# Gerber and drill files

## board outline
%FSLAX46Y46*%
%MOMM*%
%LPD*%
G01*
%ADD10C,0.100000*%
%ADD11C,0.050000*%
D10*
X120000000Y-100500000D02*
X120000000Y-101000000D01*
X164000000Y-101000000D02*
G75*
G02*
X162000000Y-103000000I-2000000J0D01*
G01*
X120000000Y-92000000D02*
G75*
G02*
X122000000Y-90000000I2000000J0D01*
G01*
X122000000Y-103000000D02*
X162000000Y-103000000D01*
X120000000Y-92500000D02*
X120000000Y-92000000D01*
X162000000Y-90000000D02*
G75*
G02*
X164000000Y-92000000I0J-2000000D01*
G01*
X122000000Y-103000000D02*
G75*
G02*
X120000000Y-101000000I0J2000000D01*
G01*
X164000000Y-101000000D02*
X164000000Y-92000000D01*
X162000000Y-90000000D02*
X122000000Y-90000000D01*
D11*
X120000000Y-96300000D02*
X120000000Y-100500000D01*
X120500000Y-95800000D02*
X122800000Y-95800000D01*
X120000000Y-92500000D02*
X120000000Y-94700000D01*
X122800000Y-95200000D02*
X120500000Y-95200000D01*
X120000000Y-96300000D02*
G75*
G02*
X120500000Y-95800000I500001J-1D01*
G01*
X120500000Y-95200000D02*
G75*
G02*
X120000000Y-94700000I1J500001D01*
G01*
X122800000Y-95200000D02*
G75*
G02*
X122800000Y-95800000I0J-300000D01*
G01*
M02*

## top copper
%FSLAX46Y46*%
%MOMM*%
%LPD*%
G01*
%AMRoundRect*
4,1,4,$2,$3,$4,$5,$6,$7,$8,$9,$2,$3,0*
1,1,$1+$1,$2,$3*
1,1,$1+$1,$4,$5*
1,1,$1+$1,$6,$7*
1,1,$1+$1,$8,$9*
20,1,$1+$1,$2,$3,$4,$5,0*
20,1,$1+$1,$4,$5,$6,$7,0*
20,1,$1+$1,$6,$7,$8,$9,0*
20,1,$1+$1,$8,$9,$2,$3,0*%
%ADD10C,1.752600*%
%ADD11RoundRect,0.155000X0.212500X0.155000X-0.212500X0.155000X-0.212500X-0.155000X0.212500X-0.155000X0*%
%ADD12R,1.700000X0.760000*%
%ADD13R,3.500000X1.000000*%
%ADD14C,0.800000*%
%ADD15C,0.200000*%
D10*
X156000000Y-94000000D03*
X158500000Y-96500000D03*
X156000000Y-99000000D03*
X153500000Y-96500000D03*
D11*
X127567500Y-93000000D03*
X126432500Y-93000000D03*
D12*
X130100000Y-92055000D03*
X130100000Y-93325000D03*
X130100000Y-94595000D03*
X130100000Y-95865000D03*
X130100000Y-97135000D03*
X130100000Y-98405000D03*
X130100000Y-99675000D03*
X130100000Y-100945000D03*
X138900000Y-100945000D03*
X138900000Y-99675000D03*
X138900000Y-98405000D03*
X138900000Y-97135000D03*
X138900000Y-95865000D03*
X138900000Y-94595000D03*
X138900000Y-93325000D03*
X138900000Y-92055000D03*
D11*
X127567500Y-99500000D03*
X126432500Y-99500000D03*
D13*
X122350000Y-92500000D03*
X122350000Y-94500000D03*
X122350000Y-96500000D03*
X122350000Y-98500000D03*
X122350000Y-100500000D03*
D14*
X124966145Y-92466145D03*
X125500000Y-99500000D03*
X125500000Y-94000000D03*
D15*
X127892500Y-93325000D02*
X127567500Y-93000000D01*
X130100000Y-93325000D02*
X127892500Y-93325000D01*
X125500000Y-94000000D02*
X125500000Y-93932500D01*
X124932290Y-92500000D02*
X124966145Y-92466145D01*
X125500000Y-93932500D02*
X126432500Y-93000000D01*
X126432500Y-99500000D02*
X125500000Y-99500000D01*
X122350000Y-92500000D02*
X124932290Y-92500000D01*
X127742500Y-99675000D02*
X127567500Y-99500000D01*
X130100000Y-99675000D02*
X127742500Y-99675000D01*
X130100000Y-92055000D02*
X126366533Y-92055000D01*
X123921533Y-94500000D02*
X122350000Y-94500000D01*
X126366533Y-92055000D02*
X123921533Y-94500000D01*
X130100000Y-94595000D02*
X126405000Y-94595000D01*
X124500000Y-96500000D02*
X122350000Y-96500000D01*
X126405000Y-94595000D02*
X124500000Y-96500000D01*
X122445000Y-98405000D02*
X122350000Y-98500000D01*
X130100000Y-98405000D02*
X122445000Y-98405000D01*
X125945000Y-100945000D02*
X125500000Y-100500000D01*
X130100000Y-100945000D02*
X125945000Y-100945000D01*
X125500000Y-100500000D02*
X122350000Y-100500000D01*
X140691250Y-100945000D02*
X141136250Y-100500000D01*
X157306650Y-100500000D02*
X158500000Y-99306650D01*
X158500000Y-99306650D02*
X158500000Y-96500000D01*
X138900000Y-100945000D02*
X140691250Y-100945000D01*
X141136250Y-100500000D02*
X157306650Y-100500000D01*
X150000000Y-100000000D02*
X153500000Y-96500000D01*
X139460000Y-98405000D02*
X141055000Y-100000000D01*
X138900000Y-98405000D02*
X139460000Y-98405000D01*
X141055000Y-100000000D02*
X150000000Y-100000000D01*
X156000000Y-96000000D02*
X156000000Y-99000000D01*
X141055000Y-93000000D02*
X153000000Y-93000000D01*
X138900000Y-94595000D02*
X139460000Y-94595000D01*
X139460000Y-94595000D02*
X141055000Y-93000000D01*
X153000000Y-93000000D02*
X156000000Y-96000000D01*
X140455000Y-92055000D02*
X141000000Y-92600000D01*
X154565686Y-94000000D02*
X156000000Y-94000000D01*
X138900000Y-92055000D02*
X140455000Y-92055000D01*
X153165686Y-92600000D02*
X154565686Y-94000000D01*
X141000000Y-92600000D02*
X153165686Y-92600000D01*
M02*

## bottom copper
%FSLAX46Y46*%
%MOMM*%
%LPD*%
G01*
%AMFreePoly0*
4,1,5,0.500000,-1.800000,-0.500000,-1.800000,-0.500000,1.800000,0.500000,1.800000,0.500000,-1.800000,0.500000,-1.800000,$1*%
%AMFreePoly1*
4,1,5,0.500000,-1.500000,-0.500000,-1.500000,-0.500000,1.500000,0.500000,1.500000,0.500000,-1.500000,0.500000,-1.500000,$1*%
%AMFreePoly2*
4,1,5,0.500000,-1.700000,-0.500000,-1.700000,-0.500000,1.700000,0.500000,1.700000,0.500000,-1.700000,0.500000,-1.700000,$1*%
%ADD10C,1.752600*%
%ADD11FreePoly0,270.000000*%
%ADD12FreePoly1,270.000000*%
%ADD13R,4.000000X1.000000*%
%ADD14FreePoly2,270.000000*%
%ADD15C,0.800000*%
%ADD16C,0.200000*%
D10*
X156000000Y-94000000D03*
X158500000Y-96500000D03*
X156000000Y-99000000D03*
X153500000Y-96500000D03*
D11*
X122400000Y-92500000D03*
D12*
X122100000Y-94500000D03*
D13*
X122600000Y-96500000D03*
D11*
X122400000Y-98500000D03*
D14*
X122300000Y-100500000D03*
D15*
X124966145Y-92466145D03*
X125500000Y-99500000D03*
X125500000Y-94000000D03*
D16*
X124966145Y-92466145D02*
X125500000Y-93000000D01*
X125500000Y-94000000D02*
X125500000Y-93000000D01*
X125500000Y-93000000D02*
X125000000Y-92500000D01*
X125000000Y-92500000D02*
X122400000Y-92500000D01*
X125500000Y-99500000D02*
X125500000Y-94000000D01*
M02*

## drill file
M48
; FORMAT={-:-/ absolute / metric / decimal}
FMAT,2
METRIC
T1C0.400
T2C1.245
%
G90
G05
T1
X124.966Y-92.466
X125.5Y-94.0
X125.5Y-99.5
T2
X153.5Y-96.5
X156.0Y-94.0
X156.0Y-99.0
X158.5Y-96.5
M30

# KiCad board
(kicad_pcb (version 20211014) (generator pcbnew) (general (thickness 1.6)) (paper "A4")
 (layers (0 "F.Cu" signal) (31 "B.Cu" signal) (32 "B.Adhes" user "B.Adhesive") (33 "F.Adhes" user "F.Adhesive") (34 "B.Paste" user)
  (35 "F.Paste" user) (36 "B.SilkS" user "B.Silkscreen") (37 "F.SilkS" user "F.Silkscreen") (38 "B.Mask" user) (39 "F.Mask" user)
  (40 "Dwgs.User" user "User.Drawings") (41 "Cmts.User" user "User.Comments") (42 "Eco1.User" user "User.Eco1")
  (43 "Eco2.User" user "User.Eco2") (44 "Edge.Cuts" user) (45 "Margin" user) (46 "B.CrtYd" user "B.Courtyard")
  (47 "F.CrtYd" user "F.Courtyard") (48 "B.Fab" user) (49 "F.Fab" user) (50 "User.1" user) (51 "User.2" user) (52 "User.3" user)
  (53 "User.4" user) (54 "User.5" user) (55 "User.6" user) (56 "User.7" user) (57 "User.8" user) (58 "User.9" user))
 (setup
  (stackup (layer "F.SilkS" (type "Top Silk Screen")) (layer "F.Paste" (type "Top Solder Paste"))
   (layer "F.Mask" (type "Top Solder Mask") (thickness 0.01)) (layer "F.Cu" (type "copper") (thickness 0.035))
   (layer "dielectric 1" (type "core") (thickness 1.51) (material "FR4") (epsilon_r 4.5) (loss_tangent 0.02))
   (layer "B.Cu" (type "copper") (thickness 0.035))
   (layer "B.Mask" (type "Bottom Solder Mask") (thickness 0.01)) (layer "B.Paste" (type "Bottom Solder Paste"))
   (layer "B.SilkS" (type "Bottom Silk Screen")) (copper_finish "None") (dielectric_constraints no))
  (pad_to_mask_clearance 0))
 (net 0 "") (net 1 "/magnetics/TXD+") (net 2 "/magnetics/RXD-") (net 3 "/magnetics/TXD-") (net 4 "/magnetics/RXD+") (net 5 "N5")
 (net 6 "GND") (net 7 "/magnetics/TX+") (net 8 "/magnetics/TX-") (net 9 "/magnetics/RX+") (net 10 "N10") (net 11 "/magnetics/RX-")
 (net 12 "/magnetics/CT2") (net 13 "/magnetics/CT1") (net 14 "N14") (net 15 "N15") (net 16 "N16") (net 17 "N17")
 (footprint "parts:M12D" (layer "F.Cu") (at 156 96.5 -90)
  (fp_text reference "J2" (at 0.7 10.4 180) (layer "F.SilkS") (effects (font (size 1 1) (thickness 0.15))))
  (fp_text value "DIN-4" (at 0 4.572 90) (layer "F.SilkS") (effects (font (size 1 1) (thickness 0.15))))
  (pad "1" thru_hole circle (at -2.5 0 270) (size 1.7526 1.7526) (drill 1.2446) (layers *.Cu *.Mask) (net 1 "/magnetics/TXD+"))
  (pad "2" thru_hole circle (at 0 -2.5 270) (size 1.7526 1.7526) (drill 1.2446) (layers *.Cu *.Mask) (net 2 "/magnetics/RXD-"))
  (pad "3" thru_hole circle (at 2.5 0) (size 1.7526 1.7526) (drill 1.2446) (layers *.Cu *.Mask) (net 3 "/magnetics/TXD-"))
  (pad "4" thru_hole circle (at 0 2.5) (size 1.7526 1.7526) (drill 1.2446) (layers *.Cu *.Mask) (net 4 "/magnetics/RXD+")))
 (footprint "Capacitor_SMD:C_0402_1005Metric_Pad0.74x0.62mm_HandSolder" (layer "F.Cu") (at 127 93 180)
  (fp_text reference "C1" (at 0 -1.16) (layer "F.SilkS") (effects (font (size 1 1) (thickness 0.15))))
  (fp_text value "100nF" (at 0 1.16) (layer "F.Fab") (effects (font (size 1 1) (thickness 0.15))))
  (pad "1" smd roundrect (at -0.5675 0 180) (size 0.735 0.62) (layers "F.Cu" "F.Paste" "F.Mask") (roundrect_rratio 0.25) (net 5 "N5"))
  (pad "2" smd roundrect (at 0.5675 0 180) (size 0.735 0.62) (layers "F.Cu" "F.Paste" "F.Mask") (roundrect_rratio 0.25) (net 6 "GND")))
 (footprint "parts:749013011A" (layer "F.Cu") (at 134.5 96.5)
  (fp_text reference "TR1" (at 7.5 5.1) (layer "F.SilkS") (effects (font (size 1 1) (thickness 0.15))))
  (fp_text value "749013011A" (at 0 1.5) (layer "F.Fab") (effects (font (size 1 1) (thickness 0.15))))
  (pad "1" smd rect (at -4.4 -4.445) (size 1.7 0.76) (layers "F.Cu" "F.Paste" "F.Mask") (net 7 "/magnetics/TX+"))
  (pad "2" smd rect (at -4.4 -3.175) (size 1.7 0.76) (layers "F.Cu" "F.Paste" "F.Mask") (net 5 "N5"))
  (pad "3" smd rect (at -4.4 -1.905) (size 1.7 0.76) (layers "F.Cu" "F.Paste" "F.Mask") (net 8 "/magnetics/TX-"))
  (pad "4" smd rect (at -4.4 -0.635) (size 1.7 0.76) (layers "F.Cu" "F.Paste" "F.Mask"))
  (pad "5" smd rect (at -4.4 0.635) (size 1.7 0.76) (layers "F.Cu" "F.Paste" "F.Mask"))
  (pad "6" smd rect (at -4.4 1.905) (size 1.7 0.76) (layers "F.Cu" "F.Paste" "F.Mask") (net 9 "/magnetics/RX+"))
  (pad "7" smd rect (at -4.4 3.175) (size 1.7 0.76) (layers "F.Cu" "F.Paste" "F.Mask") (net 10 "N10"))
  (pad "8" smd rect (at -4.4 4.445) (size 1.7 0.76) (layers "F.Cu" "F.Paste" "F.Mask") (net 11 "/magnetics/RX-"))
  (pad "9" smd rect (at 4.4 4.445) (size 1.7 0.76) (layers "F.Cu" "F.Paste" "F.Mask") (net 2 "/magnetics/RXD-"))
  (pad "10" smd rect (at 4.4 3.175) (size 1.7 0.76) (layers "F.Cu" "F.Paste" "F.Mask") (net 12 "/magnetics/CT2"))
  (pad "11" smd rect (at 4.4 1.905) (size 1.7 0.76) (layers "F.Cu" "F.Paste" "F.Mask") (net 4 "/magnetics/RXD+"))
  (pad "12" smd rect (at 4.4 0.635) (size 1.7 0.76) (layers "F.Cu" "F.Paste" "F.Mask"))
  (pad "13" smd rect (at 4.4 -0.635) (size 1.7 0.76) (layers "F.Cu" "F.Paste" "F.Mask"))
  (pad "14" smd rect (at 4.4 -1.905) (size 1.7 0.76) (layers "F.Cu" "F.Paste" "F.Mask") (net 3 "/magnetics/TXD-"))
  (pad "15" smd rect (at 4.4 -3.175) (size 1.7 0.76) (layers "F.Cu" "F.Paste" "F.Mask") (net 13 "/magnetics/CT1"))
  (pad "16" smd rect (at 4.4 -4.445) (size 1.7 0.76) (layers "F.Cu" "F.Paste" "F.Mask") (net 1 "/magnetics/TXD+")))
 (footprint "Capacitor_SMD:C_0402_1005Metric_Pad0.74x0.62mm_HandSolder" (layer "F.Cu") (at 127 99.5 180)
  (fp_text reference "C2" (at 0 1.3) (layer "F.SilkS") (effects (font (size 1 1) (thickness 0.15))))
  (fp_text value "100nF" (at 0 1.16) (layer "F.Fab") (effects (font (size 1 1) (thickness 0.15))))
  (pad "1" smd roundrect (at -0.5675 0 180) (size 0.735 0.62) (layers "F.Cu" "F.Paste" "F.Mask") (roundrect_rratio 0.25) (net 10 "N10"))
  (pad "2" smd roundrect (at 0.5675 0 180) (size 0.735 0.62) (layers "F.Cu" "F.Paste" "F.Mask") (roundrect_rratio 0.25) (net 6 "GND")))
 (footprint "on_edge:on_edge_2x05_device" (layer "F.Cu") (at 120 96.5 -90)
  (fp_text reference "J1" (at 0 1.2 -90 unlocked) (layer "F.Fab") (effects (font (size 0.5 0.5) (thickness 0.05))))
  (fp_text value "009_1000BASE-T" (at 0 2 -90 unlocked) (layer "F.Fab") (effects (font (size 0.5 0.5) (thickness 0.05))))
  (fp_line (start -0.2 0) (end 4 0) (layer "Edge.Cuts") (width 0.05))
  (fp_line (start -0.7 -0.5) (end -0.7 -2.8) (layer "Edge.Cuts") (width 0.05))
  (fp_line (start -4 0) (end -1.8 0) (layer "Edge.Cuts") (width 0.05))
  (fp_line (start -1.3 -2.8) (end -1.3 -0.5) (layer "Edge.Cuts") (width 0.05))
  (fp_arc (start -0.2 0) (mid -0.553553 -0.146447) (end -0.7 -0.5) (layer "Edge.Cuts") (width 0.05))
  (fp_arc (start -1.3 -0.5) (mid -1.446447 -0.146447) (end -1.8 0) (layer "Edge.Cuts") (width 0.05))
  (fp_arc (start -1.3 -2.8) (mid -1 -3.1) (end -0.7 -2.8) (layer "Edge.Cuts") (width 0.05))
  (pad "1" smd rect (at -4 -2.35 90) (size 1 3.5) (layers "F.Cu" "F.Mask") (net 6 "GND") (zone_connect 0))
  (pad "2" smd rect (at -2 -2.35 270) (size 1 3.5) (layers "F.Cu" "F.Mask") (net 7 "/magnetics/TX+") (zone_connect 0))
  (pad "3" smd rect (at 0 -2.35 270) (size 1 3.5) (layers "F.Cu" "F.Mask") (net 8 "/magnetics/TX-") (zone_connect 0))
  (pad "4" smd rect (at 2 -2.35 90) (size 1 3.5) (layers "F.Cu" "F.Mask") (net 9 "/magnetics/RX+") (zone_connect 0))
  (pad "5" smd rect (at 4 -2.35 90) (size 1 3.5) (layers "F.Cu" "F.Mask") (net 11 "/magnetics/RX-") (zone_connect 0))
  (pad "6" smd custom (at -4 -2.4 270) (size 1 3.6) (layers "B.Cu" "B.Mask") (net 6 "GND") (zone_connect 0)
   (options (clearance outline) (anchor rect)) (primitives))
  (pad "7" smd custom (at -2 -2.1 270) (size 1 3) (layers "B.Cu" "B.Mask") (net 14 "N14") (zone_connect 0)
   (options (clearance outline) (anchor rect)) (primitives))
  (pad "8" smd rect (at 0 -2.6 270) (size 1 4) (layers "B.Cu" "B.Mask") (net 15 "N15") (zone_connect 0))
  (pad "9" smd custom (at 2 -2.4 270) (size 1 3.6) (layers "B.Cu" "B.Mask") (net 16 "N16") (zone_connect 0)
   (options (clearance outline) (anchor rect)) (primitives))
  (pad "10" smd custom (at 4 -2.3 270) (size 1 3.4) (layers "B.Cu" "B.Mask") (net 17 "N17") (zone_connect 0)
   (options (clearance outline) (anchor rect)) (primitives)))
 (gr_line (start 120 100.5) (end 120 101) (layer "Edge.Cuts") (width 0.1))
 (gr_arc (start 164 101) (mid 163.414214 102.414214) (end 162 103) (layer "Edge.Cuts") (width 0.1))
 (gr_arc (start 120 92) (mid 120.585786 90.585786) (end 122 90) (layer "Edge.Cuts") (width 0.1))
 (gr_line (start 122 103) (end 162 103) (layer "Edge.Cuts") (width 0.1))
 (gr_line (start 120 92.5) (end 120 92) (layer "Edge.Cuts") (width 0.1))
 (gr_arc (start 162 90) (mid 163.414214 90.585786) (end 164 92) (layer "Edge.Cuts") (width 0.1))
 (gr_arc (start 122 103) (mid 120.585786 102.414214) (end 120 101) (layer "Edge.Cuts") (width 0.1))
 (gr_line (start 164 101) (end 164 92) (layer "Edge.Cuts") (width 0.1))
 (gr_line (start 162 90) (end 122 90) (layer "Edge.Cuts") (width 0.1))
 (segment (start 127.8925 93.325) (end 127.5675 93) (width 0.2) (layer "F.Cu") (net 5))
 (segment (start 130.1 93.325) (end 127.8925 93.325) (width 0.2) (layer "F.Cu") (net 5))
 (segment (start 125.5 94) (end 125.5 93.9325) (width 0.2) (layer "F.Cu") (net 6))
 (segment (start 124.93229 92.5) (end 124.966145 92.466145) (width 0.2) (layer "F.Cu") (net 6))
 (segment (start 125.5 93.9325) (end 126.4325 93) (width 0.2) (layer "F.Cu") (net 6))
 (segment (start 126.4325 99.5) (end 125.5 99.5) (width 0.2) (layer "F.Cu") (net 6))
 (segment (start 122.35 92.5) (end 124.93229 92.5) (width 0.2) (layer "F.Cu") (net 6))
 (via (at 124.966145 92.466145) (size 0.8) (drill 0.4) (layers "F.Cu" "B.Cu") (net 6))
 (via (at 125.5 99.5) (size 0.8) (drill 0.4) (layers "F.Cu" "B.Cu") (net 6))
 (via (at 125.5 94) (size 0.8) (drill 0.4) (layers "F.Cu" "B.Cu") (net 6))
 (segment (start 124.966145 92.466145) (end 125.5 93) (width 0.2) (layer "B.Cu") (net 6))
 (segment (start 125.5 94) (end 125.5 93) (width 0.2) (layer "B.Cu") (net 6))
 (segment (start 125.5 93) (end 125 92.5) (width 0.2) (layer "B.Cu") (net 6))
 (segment (start 125 92.5) (end 122.4 92.5) (width 0.2) (layer "B.Cu") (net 6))
 (segment (start 125.5 99.5) (end 125.5 94) (width 0.2) (layer "B.Cu") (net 6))
 (segment (start 127.7425 99.675) (end 127.5675 99.5) (width 0.2) (layer "F.Cu") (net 10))
 (segment (start 130.1 99.675) (end 127.7425 99.675) (width 0.2) (layer "F.Cu") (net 10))
 (segment (start 130.1 92.055) (end 126.366533 92.055) (width 0.2) (layer "F.Cu") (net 7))
 (segment (start 123.921533 94.5) (end 122.35 94.5) (width 0.2) (layer "F.Cu") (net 7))
 (segment (start 126.366533 92.055) (end 123.921533 94.5) (width 0.2) (layer "F.Cu") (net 7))
 (segment (start 130.1 94.595) (end 126.405 94.595) (width 0.2) (layer "F.Cu") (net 8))
 (segment (start 124.5 96.5) (end 122.35 96.5) (width 0.2) (layer "F.Cu") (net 8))
 (segment (start 126.405 94.595) (end 124.5 96.5) (width 0.2) (layer "F.Cu") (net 8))
 (segment (start 122.445 98.405) (end 122.35 98.5) (width 0.2) (layer "F.Cu") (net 9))
 (segment (start 130.1 98.405) (end 122.445 98.405) (width 0.2) (layer "F.Cu") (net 9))
 (segment (start 125.945 100.945) (end 125.5 100.5) (width 0.2) (layer "F.Cu") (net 11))
 (segment (start 130.1 100.945) (end 125.945 100.945) (width 0.2) (layer "F.Cu") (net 11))
 (segment (start 125.5 100.5) (end 122.35 100.5) (width 0.2) (layer "F.Cu") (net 11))
 (segment (start 140.69125 100.945) (end 141.13625 100.5) (width 0.2) (layer "F.Cu") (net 2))
 (segment (start 157.30665 100.5) (end 158.5 99.30665) (width 0.2) (layer "F.Cu") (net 2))
 (segment (start 158.5 99.30665) (end 158.5 96.5) (width 0.2) (layer "F.Cu") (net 2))
 (segment (start 138.9 100.945) (end 140.69125 100.945) (width 0.2) (layer "F.Cu") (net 2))
 (segment (start 141.13625 100.5) (end 157.30665 100.5) (width 0.2) (layer "F.Cu") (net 2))
 (segment (start 150 100) (end 153.5 96.5) (width 0.2) (layer "F.Cu") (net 4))
 (segment (start 139.46 98.405) (end 141.055 100) (width 0.2) (layer "F.Cu") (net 4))
 (segment (start 138.9 98.405) (end 139.46 98.405) (width 0.2) (layer "F.Cu") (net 4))
 (segment (start 141.055 100) (end 150 100) (width 0.2) (layer "F.Cu") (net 4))
 (segment (start 156 96) (end 156 99) (width 0.2) (layer "F.Cu") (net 3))
 (segment (start 141.055 93) (end 153 93) (width 0.2) (layer "F.Cu") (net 3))
 (segment (start 138.9 94.595) (end 139.46 94.595) (width 0.2) (layer "F.Cu") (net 3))
 (segment (start 139.46 94.595) (end 141.055 93) (width 0.2) (layer "F.Cu") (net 3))
 (segment (start 153 93) (end 156 96) (width 0.2) (layer "F.Cu") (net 3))
 (segment (start 140.455 92.055) (end 141 92.6) (width 0.2) (layer "F.Cu") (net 1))
 (segment (start 154.565686 94) (end 156 94) (width 0.2) (layer "F.Cu") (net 1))
 (segment (start 138.9 92.055) (end 140.455 92.055) (width 0.2) (layer "F.Cu") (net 1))
 (segment (start 153.165686 92.6) (end 154.565686 94) (width 0.2) (layer "F.Cu") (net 1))
 (segment (start 141 92.6) (end 153.165686 92.6) (width 0.2) (layer "F.Cu") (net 1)))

